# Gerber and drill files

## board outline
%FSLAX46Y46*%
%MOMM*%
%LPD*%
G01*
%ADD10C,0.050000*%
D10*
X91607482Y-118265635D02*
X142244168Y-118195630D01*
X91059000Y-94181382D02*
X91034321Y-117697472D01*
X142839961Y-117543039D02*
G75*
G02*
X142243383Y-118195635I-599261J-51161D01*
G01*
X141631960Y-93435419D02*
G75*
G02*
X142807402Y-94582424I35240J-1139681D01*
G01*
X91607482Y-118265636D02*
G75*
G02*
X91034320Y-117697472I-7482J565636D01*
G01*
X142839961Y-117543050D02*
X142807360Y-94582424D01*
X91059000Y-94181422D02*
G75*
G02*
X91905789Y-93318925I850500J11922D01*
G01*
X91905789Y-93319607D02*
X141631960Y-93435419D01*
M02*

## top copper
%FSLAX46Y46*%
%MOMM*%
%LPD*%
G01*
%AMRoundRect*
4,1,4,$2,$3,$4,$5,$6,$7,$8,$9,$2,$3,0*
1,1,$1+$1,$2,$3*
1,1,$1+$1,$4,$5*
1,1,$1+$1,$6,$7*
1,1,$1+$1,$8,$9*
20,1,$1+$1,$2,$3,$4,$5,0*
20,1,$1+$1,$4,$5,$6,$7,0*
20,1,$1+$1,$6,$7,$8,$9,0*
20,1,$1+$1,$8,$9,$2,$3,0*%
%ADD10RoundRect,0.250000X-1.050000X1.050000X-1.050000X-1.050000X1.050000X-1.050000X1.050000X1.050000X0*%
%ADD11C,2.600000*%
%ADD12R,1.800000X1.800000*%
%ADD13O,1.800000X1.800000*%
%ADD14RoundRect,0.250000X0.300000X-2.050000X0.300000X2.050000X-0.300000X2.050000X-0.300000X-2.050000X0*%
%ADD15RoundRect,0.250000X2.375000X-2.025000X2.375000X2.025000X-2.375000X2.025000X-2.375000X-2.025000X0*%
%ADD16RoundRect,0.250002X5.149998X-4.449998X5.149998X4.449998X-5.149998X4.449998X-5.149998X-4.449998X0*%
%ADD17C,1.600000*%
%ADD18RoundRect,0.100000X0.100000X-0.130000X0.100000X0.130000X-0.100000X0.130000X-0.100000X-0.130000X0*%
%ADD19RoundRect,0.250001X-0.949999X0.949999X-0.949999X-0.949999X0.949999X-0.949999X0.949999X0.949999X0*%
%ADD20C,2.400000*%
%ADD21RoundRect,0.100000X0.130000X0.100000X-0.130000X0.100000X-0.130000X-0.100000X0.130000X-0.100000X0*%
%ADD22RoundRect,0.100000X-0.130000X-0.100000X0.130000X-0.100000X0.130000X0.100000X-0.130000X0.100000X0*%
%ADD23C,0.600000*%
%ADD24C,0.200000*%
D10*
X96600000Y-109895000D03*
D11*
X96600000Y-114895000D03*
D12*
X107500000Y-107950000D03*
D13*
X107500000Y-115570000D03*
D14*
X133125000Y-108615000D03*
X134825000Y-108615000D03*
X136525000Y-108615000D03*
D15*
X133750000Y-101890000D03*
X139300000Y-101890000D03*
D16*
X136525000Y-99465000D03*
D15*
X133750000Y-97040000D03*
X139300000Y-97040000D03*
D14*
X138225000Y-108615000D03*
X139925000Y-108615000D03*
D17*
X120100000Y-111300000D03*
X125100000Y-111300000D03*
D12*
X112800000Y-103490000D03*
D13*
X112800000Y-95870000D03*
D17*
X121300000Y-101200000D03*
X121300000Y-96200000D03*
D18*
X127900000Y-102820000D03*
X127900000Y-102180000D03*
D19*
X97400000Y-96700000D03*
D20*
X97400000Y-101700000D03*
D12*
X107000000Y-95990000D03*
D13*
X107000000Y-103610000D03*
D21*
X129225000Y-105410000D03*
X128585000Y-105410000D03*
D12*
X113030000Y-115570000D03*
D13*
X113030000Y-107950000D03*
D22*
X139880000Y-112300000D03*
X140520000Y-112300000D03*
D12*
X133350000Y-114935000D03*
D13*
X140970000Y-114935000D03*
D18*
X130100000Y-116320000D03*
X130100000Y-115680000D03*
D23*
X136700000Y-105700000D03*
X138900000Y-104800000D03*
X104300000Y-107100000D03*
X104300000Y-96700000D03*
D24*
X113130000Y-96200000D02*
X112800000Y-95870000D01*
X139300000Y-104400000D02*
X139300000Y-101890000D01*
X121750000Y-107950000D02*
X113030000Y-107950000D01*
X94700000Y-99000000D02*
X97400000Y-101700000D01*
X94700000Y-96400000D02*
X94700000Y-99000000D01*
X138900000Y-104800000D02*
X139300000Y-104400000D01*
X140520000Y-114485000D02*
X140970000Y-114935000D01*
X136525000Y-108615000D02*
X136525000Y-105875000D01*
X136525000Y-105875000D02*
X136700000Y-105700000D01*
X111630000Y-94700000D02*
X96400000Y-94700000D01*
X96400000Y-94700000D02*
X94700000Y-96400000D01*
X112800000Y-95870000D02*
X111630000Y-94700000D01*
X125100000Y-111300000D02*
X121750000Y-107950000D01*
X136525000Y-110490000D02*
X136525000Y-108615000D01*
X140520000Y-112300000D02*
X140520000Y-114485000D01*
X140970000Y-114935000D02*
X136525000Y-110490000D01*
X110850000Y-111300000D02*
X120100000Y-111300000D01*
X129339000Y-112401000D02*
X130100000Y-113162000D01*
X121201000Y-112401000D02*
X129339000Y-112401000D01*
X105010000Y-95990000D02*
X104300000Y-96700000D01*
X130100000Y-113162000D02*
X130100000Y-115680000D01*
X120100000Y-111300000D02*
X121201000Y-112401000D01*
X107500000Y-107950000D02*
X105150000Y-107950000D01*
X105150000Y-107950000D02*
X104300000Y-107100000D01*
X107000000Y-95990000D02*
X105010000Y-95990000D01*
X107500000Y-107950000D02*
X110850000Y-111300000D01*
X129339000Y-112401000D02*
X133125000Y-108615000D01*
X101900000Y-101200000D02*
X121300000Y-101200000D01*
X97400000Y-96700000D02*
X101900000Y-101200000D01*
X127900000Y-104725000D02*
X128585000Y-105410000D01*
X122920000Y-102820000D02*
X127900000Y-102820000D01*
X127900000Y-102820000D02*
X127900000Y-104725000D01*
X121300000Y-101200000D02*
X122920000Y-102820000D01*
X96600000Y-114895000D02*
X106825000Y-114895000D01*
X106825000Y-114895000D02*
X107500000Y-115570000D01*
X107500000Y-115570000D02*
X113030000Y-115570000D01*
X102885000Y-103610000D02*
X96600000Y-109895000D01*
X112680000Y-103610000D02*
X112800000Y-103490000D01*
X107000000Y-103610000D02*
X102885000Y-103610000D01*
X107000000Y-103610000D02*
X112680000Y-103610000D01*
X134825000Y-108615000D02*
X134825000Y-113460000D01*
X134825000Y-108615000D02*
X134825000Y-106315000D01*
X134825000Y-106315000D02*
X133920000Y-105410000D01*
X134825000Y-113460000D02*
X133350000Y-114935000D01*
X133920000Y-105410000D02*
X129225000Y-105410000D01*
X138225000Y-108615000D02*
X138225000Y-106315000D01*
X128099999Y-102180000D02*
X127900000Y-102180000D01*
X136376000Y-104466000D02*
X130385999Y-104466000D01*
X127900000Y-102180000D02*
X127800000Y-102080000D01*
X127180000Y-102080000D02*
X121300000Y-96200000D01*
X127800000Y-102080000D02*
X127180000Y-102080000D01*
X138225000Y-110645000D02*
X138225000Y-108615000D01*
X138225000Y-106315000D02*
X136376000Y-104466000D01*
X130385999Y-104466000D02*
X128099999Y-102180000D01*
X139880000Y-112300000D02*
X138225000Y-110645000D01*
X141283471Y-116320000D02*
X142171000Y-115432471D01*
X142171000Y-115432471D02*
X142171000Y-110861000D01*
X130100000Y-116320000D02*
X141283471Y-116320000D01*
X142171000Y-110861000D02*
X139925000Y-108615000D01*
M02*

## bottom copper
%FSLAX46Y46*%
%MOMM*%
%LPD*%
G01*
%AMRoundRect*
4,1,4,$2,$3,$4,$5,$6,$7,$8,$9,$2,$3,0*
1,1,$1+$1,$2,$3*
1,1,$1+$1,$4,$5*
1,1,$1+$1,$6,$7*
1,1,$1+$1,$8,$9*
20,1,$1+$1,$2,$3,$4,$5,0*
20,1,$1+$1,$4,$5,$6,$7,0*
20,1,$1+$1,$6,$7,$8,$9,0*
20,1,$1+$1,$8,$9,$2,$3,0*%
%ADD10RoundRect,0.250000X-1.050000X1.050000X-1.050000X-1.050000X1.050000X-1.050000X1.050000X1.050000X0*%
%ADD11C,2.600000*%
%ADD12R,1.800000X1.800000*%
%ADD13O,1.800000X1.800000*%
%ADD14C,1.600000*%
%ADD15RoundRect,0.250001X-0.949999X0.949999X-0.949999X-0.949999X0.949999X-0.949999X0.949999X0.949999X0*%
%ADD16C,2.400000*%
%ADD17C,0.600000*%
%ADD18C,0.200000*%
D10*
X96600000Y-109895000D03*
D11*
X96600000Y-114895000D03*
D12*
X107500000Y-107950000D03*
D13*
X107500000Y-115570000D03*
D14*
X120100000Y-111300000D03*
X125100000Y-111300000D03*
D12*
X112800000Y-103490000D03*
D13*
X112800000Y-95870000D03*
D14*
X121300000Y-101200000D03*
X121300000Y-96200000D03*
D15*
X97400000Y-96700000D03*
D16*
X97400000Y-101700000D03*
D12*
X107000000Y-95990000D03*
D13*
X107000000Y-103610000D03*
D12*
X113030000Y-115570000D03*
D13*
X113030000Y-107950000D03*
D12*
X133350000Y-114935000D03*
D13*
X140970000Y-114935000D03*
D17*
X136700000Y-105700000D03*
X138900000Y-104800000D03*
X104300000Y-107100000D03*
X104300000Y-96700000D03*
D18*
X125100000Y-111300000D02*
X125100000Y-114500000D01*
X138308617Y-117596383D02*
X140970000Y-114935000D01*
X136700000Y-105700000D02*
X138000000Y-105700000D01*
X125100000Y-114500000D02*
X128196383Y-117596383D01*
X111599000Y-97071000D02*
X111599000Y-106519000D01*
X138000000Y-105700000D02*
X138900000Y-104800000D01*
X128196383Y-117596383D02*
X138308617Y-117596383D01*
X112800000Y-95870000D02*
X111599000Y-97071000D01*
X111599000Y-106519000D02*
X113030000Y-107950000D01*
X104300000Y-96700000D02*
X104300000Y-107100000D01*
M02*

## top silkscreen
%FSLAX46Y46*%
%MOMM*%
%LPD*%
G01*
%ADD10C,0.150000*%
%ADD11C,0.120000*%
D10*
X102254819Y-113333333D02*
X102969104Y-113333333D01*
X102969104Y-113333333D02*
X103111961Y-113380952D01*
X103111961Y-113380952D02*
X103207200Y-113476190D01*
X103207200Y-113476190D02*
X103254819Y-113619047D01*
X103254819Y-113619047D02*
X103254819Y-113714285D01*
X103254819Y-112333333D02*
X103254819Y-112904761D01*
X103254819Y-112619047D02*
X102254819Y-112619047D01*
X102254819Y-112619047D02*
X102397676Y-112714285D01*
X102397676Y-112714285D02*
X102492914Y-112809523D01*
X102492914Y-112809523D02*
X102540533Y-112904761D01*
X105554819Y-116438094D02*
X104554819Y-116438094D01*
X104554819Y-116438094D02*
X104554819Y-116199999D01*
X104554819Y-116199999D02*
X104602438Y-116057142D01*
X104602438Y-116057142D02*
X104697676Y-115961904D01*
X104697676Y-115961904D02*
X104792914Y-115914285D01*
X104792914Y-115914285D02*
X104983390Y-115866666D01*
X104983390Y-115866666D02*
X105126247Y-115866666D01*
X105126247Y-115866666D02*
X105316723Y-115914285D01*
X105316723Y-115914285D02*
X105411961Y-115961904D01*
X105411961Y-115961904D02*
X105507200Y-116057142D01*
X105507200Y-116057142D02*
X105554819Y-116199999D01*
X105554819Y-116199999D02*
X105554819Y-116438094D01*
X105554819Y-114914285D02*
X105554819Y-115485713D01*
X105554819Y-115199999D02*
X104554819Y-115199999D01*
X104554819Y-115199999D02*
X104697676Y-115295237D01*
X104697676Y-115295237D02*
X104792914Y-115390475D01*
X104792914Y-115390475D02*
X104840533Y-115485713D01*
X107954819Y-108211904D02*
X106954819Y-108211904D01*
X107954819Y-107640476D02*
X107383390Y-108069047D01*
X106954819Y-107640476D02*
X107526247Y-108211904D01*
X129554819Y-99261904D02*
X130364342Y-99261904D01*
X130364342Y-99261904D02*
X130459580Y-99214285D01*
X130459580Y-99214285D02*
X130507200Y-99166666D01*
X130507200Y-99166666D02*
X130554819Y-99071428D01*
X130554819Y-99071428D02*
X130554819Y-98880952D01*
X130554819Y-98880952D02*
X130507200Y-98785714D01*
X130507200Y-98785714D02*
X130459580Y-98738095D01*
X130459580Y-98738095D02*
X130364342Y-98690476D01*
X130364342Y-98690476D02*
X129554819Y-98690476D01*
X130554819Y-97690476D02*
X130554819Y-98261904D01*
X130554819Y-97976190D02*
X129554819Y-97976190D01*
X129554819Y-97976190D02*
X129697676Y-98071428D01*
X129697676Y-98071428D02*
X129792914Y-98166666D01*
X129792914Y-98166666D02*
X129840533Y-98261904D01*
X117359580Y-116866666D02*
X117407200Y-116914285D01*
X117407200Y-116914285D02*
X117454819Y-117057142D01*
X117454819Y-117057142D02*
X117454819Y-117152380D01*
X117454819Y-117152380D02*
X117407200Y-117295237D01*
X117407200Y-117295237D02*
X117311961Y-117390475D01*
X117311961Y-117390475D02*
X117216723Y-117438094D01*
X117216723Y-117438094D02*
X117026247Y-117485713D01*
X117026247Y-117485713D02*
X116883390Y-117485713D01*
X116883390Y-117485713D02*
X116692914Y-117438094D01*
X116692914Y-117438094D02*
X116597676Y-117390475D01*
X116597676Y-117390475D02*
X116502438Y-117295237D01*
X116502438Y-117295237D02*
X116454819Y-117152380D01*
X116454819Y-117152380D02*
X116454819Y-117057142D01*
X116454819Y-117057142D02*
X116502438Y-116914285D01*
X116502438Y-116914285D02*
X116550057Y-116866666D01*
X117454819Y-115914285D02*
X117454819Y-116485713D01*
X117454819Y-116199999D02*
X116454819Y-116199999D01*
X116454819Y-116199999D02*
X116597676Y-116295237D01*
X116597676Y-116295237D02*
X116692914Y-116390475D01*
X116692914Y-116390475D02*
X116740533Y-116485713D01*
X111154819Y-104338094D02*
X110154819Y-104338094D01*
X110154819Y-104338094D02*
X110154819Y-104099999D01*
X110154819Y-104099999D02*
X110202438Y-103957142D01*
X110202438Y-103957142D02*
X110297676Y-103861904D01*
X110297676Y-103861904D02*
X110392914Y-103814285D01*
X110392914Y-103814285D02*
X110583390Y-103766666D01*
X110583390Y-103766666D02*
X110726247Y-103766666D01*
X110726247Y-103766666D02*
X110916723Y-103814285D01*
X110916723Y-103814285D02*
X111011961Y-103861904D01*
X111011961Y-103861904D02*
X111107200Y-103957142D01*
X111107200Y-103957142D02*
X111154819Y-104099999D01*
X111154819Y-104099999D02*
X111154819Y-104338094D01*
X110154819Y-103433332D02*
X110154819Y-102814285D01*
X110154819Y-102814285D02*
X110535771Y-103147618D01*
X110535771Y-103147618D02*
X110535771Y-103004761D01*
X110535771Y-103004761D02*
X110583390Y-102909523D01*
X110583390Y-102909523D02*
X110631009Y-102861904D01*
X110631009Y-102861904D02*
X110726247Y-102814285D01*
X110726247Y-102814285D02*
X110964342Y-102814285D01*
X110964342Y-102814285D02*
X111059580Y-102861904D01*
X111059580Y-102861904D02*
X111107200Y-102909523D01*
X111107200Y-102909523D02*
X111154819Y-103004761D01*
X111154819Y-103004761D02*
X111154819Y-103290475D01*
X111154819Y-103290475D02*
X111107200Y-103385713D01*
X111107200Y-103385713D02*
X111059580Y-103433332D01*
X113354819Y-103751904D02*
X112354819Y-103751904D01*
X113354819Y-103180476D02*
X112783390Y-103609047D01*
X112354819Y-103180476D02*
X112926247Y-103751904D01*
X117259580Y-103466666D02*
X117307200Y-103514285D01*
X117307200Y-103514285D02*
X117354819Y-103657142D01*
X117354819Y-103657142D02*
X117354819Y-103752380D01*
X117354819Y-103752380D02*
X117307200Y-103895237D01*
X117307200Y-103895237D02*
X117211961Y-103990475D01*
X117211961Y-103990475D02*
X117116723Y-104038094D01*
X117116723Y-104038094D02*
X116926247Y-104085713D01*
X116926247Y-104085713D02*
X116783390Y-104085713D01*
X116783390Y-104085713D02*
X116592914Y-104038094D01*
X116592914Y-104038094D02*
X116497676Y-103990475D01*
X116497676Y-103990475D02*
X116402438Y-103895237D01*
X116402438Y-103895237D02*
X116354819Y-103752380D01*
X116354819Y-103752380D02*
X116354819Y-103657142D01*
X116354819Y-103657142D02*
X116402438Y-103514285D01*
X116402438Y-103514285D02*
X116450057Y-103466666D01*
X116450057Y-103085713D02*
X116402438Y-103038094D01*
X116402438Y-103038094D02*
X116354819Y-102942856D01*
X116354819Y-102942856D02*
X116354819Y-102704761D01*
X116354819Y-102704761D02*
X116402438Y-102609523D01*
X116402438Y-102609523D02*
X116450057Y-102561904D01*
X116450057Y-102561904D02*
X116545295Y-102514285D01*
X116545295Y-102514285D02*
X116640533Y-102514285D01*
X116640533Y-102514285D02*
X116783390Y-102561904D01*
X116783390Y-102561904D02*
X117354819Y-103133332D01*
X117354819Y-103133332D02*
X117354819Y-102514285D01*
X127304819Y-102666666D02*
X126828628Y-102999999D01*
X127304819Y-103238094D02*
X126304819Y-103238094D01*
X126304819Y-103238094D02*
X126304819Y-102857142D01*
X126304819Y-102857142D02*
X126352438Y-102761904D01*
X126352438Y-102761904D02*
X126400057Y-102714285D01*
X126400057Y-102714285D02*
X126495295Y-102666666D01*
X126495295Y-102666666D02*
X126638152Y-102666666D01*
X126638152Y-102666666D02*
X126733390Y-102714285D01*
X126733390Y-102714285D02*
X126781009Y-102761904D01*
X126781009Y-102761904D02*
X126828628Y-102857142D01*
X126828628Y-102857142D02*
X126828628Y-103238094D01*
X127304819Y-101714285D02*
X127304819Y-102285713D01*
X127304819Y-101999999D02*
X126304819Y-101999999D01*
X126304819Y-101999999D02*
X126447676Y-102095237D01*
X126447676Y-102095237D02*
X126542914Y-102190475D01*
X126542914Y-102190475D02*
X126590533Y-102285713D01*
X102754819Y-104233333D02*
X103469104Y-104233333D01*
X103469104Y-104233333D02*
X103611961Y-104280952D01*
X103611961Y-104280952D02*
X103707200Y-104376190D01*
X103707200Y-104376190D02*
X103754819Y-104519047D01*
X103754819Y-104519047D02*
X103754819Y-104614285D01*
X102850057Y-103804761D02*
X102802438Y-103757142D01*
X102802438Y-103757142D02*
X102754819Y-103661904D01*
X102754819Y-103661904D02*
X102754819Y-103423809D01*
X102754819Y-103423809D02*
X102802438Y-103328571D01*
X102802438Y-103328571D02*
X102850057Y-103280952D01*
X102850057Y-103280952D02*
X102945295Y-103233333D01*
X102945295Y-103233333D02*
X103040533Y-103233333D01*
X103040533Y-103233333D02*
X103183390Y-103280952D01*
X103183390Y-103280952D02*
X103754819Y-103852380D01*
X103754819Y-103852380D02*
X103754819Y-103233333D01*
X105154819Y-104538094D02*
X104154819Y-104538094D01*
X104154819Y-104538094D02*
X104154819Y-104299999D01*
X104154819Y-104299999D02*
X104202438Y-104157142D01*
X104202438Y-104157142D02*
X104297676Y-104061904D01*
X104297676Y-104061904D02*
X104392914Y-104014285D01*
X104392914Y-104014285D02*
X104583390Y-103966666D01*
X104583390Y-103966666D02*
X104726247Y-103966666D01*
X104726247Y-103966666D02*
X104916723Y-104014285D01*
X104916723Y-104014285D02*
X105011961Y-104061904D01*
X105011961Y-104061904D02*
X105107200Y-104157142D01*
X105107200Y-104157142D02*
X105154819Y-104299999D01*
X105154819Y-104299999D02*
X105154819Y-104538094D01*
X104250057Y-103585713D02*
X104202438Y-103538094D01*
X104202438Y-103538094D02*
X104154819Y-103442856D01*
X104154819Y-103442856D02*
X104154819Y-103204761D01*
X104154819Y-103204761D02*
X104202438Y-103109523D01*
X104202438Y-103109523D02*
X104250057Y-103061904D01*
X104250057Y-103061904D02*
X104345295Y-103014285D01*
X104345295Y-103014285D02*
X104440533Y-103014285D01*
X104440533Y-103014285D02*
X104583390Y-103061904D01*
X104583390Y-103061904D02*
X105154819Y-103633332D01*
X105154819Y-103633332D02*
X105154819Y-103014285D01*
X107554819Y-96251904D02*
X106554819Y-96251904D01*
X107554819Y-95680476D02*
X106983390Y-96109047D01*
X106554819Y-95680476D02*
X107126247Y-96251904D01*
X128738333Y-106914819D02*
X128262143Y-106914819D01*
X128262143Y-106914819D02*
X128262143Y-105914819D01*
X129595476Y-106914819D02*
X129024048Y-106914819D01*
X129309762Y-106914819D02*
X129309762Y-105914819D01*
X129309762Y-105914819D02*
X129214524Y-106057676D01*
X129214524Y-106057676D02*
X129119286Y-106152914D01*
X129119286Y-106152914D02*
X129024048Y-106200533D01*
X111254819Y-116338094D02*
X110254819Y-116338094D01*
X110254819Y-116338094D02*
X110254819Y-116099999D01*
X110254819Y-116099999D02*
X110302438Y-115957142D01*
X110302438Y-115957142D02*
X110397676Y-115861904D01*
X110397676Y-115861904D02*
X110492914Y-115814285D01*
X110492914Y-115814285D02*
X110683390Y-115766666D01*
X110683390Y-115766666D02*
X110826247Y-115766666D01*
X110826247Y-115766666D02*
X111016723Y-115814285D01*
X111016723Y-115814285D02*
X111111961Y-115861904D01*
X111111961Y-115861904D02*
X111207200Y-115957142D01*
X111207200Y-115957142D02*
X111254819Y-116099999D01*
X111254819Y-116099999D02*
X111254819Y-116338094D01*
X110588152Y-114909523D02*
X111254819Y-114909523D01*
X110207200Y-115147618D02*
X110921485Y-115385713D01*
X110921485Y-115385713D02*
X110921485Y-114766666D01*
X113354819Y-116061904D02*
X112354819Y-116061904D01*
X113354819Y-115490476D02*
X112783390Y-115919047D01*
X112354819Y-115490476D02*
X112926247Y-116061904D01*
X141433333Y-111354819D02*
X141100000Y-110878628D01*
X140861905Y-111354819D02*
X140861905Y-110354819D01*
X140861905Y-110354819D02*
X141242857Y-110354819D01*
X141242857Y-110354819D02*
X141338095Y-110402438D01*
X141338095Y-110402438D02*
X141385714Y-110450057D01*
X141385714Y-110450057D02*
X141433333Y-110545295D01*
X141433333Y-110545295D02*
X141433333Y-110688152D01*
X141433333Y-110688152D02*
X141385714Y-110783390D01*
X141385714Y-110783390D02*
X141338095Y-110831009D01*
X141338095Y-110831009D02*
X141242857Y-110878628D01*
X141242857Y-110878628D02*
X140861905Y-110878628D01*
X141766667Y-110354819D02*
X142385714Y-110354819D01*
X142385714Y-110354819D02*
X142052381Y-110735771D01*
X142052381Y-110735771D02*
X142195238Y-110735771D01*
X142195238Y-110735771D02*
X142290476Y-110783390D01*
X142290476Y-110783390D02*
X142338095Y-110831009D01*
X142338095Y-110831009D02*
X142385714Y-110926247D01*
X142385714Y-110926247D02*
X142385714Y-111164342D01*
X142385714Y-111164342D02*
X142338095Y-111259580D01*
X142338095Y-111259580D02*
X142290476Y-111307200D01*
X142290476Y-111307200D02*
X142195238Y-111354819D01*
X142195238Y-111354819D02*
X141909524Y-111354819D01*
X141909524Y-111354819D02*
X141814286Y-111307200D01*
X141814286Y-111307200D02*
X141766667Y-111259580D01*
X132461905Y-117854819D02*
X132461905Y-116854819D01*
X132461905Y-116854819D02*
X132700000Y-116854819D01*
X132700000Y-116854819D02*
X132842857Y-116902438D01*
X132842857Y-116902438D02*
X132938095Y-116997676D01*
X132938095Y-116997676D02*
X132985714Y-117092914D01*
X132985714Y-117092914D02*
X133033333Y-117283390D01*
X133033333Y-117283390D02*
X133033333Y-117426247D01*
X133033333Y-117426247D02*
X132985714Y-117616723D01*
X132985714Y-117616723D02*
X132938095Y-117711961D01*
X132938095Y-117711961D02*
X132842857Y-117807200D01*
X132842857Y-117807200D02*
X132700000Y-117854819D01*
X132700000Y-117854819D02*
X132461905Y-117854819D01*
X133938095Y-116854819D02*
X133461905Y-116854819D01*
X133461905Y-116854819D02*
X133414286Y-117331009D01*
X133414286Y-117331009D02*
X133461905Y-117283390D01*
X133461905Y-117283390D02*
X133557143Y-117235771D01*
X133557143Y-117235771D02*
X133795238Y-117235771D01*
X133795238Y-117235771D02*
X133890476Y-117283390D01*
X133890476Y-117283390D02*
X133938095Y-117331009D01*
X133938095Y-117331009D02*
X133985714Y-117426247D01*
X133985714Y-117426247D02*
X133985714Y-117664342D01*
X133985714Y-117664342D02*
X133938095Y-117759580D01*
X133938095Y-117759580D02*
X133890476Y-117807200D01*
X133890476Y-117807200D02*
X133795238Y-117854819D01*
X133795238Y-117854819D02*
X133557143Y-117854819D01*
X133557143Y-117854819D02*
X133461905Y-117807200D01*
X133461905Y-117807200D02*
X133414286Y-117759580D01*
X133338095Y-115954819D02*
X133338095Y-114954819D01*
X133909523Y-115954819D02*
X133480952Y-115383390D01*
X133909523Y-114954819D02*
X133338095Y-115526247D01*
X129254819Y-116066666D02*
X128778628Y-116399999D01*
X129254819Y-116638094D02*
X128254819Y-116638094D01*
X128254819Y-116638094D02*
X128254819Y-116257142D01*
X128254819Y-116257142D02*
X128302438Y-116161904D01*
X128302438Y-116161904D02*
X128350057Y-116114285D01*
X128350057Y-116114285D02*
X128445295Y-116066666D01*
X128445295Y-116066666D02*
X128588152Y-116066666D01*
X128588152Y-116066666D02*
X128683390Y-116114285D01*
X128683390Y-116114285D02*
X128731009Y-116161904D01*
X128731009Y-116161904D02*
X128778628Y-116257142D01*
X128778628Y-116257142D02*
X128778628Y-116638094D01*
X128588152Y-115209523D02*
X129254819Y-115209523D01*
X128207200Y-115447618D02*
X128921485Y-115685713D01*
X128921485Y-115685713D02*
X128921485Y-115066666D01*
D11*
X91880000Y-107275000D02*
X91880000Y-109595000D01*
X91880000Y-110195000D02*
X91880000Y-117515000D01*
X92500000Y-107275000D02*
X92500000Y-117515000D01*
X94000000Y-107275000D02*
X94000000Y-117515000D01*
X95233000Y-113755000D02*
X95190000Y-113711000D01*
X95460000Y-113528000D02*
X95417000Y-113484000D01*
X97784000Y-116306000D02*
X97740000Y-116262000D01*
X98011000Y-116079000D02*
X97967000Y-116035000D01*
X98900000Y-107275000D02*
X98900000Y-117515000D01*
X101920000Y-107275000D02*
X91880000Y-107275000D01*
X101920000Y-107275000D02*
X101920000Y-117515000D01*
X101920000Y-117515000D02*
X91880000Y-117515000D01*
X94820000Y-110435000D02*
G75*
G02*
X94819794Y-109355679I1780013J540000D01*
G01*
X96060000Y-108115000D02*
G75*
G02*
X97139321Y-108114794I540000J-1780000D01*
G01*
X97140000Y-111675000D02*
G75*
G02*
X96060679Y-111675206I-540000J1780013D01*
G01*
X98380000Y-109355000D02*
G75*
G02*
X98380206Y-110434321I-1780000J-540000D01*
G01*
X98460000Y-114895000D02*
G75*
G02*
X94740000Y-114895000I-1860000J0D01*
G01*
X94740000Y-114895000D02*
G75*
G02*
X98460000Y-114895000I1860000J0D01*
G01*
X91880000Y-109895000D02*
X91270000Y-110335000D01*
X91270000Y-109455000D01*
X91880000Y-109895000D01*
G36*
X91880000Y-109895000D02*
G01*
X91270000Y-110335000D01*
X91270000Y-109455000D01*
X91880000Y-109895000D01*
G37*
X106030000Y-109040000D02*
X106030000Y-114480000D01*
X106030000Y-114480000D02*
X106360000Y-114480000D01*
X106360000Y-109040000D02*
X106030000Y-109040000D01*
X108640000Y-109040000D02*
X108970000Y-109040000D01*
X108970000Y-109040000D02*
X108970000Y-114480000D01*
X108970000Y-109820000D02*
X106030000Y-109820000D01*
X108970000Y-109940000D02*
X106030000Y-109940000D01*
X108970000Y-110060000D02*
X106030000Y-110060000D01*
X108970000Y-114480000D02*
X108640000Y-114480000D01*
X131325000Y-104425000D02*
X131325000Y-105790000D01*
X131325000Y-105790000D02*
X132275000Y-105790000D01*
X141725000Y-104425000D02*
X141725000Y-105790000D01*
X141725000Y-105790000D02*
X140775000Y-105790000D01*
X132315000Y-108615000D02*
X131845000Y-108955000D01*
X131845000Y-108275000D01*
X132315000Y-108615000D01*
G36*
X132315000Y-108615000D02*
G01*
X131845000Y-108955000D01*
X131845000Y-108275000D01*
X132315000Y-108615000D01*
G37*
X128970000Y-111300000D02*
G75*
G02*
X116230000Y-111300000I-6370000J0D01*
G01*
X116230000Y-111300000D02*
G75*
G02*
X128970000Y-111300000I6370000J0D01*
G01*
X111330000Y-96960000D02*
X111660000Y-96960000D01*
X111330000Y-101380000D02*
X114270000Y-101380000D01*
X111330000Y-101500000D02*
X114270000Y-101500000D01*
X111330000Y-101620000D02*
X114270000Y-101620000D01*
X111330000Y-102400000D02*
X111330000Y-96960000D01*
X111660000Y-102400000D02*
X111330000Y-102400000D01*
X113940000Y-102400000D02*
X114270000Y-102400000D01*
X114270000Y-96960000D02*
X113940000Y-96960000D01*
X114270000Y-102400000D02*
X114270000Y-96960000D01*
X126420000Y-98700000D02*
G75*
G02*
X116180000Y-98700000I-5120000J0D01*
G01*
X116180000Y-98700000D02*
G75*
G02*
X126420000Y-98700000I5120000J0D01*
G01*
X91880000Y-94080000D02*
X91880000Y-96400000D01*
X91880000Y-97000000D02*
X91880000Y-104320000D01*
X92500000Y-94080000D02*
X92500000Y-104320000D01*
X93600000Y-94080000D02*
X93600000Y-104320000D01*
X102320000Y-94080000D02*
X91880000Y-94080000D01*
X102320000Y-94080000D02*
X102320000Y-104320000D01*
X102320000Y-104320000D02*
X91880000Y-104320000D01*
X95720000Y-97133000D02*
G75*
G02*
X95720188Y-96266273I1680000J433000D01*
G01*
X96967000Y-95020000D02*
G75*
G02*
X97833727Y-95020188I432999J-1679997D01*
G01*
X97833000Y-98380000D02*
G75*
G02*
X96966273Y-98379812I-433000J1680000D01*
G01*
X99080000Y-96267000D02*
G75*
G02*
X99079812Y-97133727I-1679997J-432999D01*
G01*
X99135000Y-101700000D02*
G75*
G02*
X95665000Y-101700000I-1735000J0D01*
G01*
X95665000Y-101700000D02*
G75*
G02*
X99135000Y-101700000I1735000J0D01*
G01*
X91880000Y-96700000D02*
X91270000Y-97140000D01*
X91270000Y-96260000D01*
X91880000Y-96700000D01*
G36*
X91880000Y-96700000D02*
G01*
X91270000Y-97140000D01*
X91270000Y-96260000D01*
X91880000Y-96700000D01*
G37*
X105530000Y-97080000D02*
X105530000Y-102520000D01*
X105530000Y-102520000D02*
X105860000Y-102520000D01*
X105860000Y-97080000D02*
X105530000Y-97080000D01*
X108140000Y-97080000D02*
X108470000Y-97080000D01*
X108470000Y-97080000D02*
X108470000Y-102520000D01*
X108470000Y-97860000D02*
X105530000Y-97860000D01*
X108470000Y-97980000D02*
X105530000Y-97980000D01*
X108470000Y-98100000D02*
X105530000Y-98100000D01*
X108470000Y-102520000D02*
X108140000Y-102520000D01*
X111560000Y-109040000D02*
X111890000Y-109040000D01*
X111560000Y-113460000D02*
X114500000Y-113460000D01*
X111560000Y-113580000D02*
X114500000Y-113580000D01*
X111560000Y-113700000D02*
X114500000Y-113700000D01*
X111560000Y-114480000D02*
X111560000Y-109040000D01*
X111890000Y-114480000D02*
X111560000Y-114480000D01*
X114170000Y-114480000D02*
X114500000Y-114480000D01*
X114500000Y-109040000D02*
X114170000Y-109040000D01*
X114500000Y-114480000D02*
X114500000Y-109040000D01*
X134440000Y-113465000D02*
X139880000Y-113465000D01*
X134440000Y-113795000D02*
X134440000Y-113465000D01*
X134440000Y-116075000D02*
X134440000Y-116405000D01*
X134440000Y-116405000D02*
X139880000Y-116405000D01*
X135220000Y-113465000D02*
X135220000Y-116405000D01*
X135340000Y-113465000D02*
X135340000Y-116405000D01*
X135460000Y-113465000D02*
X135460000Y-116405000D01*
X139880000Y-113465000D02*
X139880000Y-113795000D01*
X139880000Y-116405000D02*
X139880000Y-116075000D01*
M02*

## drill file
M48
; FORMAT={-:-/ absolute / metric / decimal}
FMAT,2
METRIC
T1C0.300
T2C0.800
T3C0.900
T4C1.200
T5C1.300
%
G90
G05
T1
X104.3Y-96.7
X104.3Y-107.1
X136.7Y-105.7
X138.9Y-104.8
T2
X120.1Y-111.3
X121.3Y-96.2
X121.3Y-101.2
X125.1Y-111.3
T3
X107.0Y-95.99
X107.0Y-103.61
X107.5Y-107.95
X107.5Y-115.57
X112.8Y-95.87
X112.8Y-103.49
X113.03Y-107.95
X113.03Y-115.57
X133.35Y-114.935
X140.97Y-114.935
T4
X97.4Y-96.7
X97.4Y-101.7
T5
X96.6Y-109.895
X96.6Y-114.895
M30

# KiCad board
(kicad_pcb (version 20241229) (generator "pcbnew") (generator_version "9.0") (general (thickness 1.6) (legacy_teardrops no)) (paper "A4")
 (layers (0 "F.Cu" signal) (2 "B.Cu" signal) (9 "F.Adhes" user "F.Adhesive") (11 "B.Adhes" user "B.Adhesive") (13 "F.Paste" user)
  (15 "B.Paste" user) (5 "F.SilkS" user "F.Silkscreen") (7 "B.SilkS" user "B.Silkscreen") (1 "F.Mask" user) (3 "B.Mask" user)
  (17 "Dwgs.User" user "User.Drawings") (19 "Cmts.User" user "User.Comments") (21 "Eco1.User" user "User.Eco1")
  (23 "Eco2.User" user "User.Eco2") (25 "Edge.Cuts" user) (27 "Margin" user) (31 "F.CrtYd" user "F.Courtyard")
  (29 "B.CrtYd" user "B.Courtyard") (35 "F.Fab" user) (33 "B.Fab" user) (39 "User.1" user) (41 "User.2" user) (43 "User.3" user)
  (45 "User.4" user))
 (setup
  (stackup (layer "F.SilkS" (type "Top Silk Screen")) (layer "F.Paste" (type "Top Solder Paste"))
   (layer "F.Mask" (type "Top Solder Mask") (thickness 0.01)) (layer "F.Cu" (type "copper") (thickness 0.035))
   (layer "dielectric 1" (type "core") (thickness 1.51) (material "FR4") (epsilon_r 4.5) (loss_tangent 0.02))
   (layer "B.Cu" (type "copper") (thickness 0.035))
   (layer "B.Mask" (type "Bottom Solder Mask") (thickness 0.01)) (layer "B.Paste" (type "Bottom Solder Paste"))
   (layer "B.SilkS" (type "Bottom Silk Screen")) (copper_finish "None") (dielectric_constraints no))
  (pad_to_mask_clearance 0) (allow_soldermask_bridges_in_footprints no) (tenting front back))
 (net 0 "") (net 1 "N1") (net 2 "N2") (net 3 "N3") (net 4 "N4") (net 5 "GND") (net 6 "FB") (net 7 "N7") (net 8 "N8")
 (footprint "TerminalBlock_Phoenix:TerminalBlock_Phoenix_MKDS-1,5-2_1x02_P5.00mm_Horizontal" (layer "F.Cu") (at 96.6 109.895 -90)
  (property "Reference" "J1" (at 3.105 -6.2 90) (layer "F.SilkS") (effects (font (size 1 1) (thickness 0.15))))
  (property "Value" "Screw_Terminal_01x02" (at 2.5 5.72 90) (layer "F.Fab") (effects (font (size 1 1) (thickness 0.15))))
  (fp_line (start -2.62 4.72) (end -0.3 4.72) (stroke (width 0.12) (type solid)) (layer "F.SilkS"))
  (fp_line (start 0.3 4.72) (end 7.62 4.72) (stroke (width 0.12) (type solid)) (layer "F.SilkS"))
  (fp_line (start -2.62 4.1) (end 7.62 4.1) (stroke (width 0.12) (type solid)) (layer "F.SilkS"))
  (fp_line (start -2.62 2.6) (end 7.62 2.6) (stroke (width 0.12) (type solid)) (layer "F.SilkS"))
  (fp_line (start 3.86 1.367) (end 3.816 1.41) (stroke (width 0.12) (type solid)) (layer "F.SilkS"))
  (fp_line (start 3.633 1.14) (end 3.589 1.183) (stroke (width 0.12) (type solid)) (layer "F.SilkS"))
  (fp_line (start 6.411 -1.184) (end 6.367 -1.14) (stroke (width 0.12) (type solid)) (layer "F.SilkS"))
  (fp_line (start 6.184 -1.411) (end 6.14 -1.367) (stroke (width 0.12) (type solid)) (layer "F.SilkS"))
  (fp_line (start -2.62 -2.3) (end 7.62 -2.3) (stroke (width 0.12) (type solid)) (layer "F.SilkS"))
  (fp_line (start -2.62 -5.32) (end -2.62 4.72) (stroke (width 0.12) (type solid)) (layer "F.SilkS"))
  (fp_line (start -2.62 -5.32) (end 7.62 -5.32) (stroke (width 0.12) (type solid)) (layer "F.SilkS"))
  (fp_line (start 7.62 -5.32) (end 7.62 4.72) (stroke (width 0.12) (type solid)) (layer "F.SilkS"))
  (fp_arc (start 0.54 1.78) (mid 0.000355 1.860107) (end -0.539321 1.780206) (stroke (width 0.12) (type solid)) (layer "F.SilkS"))
  (fp_arc (start -1.78 0.54) (mid -1.860107 0.000355) (end -1.780206 -0.539321) (stroke (width 0.12) (type solid)) (layer "F.SilkS"))
  (fp_arc (start 1.78 -0.54) (mid 1.860107 -0.000355) (end 1.780206 0.539321) (stroke (width 0.12) (type solid)) (layer "F.SilkS"))
  (fp_arc (start -0.54 -1.78) (mid -0.000355 -1.860107) (end 0.539321 -1.780206) (stroke (width 0.12) (type solid)) (layer "F.SilkS"))
  (fp_circle (center 5 0) (end 6.86 0) (stroke (width 0.12) (type solid)) (fill no) (layer "F.SilkS"))
  (fp_poly (pts (xy 0 4.72) (xy 0.44 5.33) (xy -0.44 5.33) (xy 0 4.72)) (stroke (width 0.12) (type solid)) (fill yes) (layer "F.SilkS"))
  (pad "1" thru_hole roundrect (at 0 0 270) (size 2.6 2.6) (drill 1.3) (layers "*.Cu" "*.Mask") (remove_unused_layers no)
   (roundrect_rratio 0.096154) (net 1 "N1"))
  (pad "2" thru_hole circle (at 5 0 270) (size 2.6 2.6) (drill 1.3) (layers "*.Cu" "*.Mask") (remove_unused_layers no) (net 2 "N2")))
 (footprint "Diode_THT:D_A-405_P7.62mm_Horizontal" (layer "F.Cu") (at 107.5 107.95 -90)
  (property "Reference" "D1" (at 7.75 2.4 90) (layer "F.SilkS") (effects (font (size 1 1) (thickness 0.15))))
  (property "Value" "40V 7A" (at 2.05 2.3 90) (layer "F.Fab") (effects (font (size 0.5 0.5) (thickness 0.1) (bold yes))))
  (fp_line (start 1.09 1.47) (end 6.53 1.47) (stroke (width 0.12) (type solid)) (layer "F.SilkS"))
  (fp_line (start 6.53 1.47) (end 6.53 1.14) (stroke (width 0.12) (type solid)) (layer "F.SilkS"))
  (fp_line (start 1.09 1.14) (end 1.09 1.47) (stroke (width 0.12) (type solid)) (layer "F.SilkS"))
  (fp_line (start 1.09 -1.14) (end 1.09 -1.47) (stroke (width 0.12) (type solid)) (layer "F.SilkS"))
  (fp_line (start 1.09 -1.47) (end 6.53 -1.47) (stroke (width 0.12) (type solid)) (layer "F.SilkS"))
  (fp_line (start 1.87 -1.47) (end 1.87 1.47) (stroke (width 0.12) (type solid)) (layer "F.SilkS"))
  (fp_line (start 1.99 -1.47) (end 1.99 1.47) (stroke (width 0.12) (type solid)) (layer "F.SilkS"))
  (fp_line (start 2.11 -1.47) (end 2.11 1.47) (stroke (width 0.12) (type solid)) (layer "F.SilkS"))
  (fp_line (start 6.53 -1.47) (end 6.53 -1.14) (stroke (width 0.12) (type solid)) (layer "F.SilkS"))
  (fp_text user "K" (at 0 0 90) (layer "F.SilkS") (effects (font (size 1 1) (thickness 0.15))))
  (pad "1" thru_hole rect (at 0 0 270) (size 1.8 1.8) (drill 0.9) (layers "*.Cu" "*.Mask") (remove_unused_layers no) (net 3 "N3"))
  (pad "2" thru_hole oval (at 7.62 0 270) (size 1.8 1.8) (drill 0.9) (layers "*.Cu" "*.Mask") (remove_unused_layers no) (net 2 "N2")))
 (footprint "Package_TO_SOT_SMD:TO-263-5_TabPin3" (layer "F.Cu") (at 136.525 100.965 90)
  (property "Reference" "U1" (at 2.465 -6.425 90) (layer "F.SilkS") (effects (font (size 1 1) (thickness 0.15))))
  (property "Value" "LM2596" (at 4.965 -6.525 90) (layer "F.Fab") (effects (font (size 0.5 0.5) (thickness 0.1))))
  (fp_line (start -3.46 -5.2) (end -4.825 -5.2) (stroke (width 0.12) (type solid)) (layer "F.SilkS"))
  (fp_line (start -4.825 -5.2) (end -4.825 -4.25) (stroke (width 0.12) (type solid)) (layer "F.SilkS"))
  (fp_line (start -3.46 5.2) (end -4.825 5.2) (stroke (width 0.12) (type solid)) (layer "F.SilkS"))
  (fp_line (start -4.825 5.2) (end -4.825 4.25) (stroke (width 0.12) (type solid)) (layer "F.SilkS"))
  (fp_poly
   (pts (xy -7.65 -4.21) (xy -7.99 -4.68) (xy -7.31 -4.68) (xy -7.65 -4.21)) (stroke (width 0.12) (type solid)) (fill yes) (layer "F.SilkS"))
  (pad "1" smd roundrect (at -7.65 -3.4 90) (size 4.6 1.1) (layers "F.Cu" "F.Mask" "F.Paste") (roundrect_rratio 0.227273) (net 3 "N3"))
  (pad "2" smd roundrect (at -7.65 -1.7 90) (size 4.6 1.1) (layers "F.Cu" "F.Mask" "F.Paste") (roundrect_rratio 0.227273) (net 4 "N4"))
  (pad "3" smd roundrect (at -7.65 0 90) (size 4.6 1.1) (layers "F.Cu" "F.Mask" "F.Paste") (roundrect_rratio 0.227273) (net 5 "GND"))
  (pad "3" smd roundrect (at -0.925 -2.775 90) (size 4.55 5.25) (layers "F.Cu" "F.Paste") (roundrect_rratio 0.054945) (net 5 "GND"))
  (pad "3" smd roundrect (at -0.925 2.775 90) (size 4.55 5.25) (layers "F.Cu" "F.Paste") (roundrect_rratio 0.054945) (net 5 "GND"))
  (pad "3" smd roundrect (at 1.5 0 90) (size 9.4 10.8) (layers "F.Cu" "F.Mask") (roundrect_rratio 0.026596) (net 5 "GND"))
  (pad "3" smd roundrect (at 3.925 -2.775 90) (size 4.55 5.25) (layers "F.Cu" "F.Paste") (roundrect_rratio 0.054945) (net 5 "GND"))
  (pad "3" smd roundrect (at 3.925 2.775 90) (size 4.55 5.25) (layers "F.Cu" "F.Paste") (roundrect_rratio 0.054945) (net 5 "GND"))
  (pad "4" smd roundrect (at -7.65 1.7 90) (size 4.6 1.1) (layers "F.Cu" "F.Mask" "F.Paste") (roundrect_rratio 0.227273) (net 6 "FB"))
  (pad "5" smd roundrect (at -7.65 3.4 90) (size 4.6 1.1) (layers "F.Cu" "F.Mask" "F.Paste") (roundrect_rratio 0.227273) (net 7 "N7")))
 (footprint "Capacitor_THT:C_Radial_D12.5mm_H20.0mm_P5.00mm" (layer "F.Cu") (at 120.1 111.3)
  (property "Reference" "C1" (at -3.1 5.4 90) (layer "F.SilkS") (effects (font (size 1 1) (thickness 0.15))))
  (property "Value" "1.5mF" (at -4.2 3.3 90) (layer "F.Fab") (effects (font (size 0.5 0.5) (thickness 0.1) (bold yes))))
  (fp_circle (center 2.5 0) (end 8.87 0) (stroke (width 0.12) (type solid)) (fill no) (layer "F.SilkS"))
  (pad "1" thru_hole circle (at 0 0) (size 1.6 1.6) (drill 0.8) (layers "*.Cu" "*.Mask") (remove_unused_layers no) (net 3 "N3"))
  (pad "2" thru_hole circle (at 5 0) (size 1.6 1.6) (drill 0.8) (layers "*.Cu" "*.Mask") (remove_unused_layers no) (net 5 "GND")))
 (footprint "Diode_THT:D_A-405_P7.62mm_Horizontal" (layer "F.Cu") (at 112.8 103.49 90)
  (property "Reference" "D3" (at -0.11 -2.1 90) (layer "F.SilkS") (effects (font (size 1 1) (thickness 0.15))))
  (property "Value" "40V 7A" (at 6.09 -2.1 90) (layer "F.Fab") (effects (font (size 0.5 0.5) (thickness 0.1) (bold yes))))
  (fp_line (start 6.53 -1.47) (end 6.53 -1.14) (stroke (width 0.12) (type solid)) (layer "F.SilkS"))
  (fp_line (start 2.11 -1.47) (end 2.11 1.47) (stroke (width 0.12) (type solid)) (layer "F.SilkS"))
  (fp_line (start 1.99 -1.47) (end 1.99 1.47) (stroke (width 0.12) (type solid)) (layer "F.SilkS"))
  (fp_line (start 1.87 -1.47) (end 1.87 1.47) (stroke (width 0.12) (type solid)) (layer "F.SilkS"))
  (fp_line (start 1.09 -1.47) (end 6.53 -1.47) (stroke (width 0.12) (type solid)) (layer "F.SilkS"))
  (fp_line (start 1.09 -1.14) (end 1.09 -1.47) (stroke (width 0.12) (type solid)) (layer "F.SilkS"))
  (fp_line (start 1.09 1.14) (end 1.09 1.47) (stroke (width 0.12) (type solid)) (layer "F.SilkS"))
  (fp_line (start 6.53 1.47) (end 6.53 1.14) (stroke (width 0.12) (type solid)) (layer "F.SilkS"))
  (fp_line (start 1.09 1.47) (end 6.53 1.47) (stroke (width 0.12) (type solid)) (layer "F.SilkS"))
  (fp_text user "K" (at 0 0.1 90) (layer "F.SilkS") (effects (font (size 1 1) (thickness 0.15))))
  (pad "1" thru_hole rect (at 0 0 90) (size 1.8 1.8) (drill 0.9) (layers "*.Cu" "*.Mask") (remove_unused_layers no) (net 1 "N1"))
  (pad "2" thru_hole oval (at 7.62 0 90) (size 1.8 1.8) (drill 0.9) (layers "*.Cu" "*.Mask") (remove_unused_layers no) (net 5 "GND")))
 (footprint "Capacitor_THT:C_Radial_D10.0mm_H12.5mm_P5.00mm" (layer "F.Cu") (at 121.3 101.2 90)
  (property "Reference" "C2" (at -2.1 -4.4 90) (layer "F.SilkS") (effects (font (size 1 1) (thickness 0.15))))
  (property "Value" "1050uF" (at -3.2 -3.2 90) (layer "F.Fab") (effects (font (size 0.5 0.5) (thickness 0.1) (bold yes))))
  (fp_circle (center 2.5 0) (end 7.62 0) (stroke (width 0.12) (type solid)) (fill no) (layer "F.SilkS"))
  (pad "1" thru_hole circle (at 0 0 90) (size 1.6 1.6) (drill 0.8) (layers "*.Cu" "*.Mask") (remove_unused_layers no) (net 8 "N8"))
  (pad "2" thru_hole circle (at 5 0 90) (size 1.6 1.6) (drill 0.8) (layers "*.Cu" "*.Mask") (remove_unused_layers no) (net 6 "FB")))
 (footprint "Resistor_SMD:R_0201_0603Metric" (layer "F.Cu") (at 127.9 102.5 90)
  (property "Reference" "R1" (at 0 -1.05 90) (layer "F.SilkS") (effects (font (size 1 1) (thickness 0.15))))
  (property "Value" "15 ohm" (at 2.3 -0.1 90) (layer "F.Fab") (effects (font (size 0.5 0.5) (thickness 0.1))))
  (pad "" smd roundrect (at -0.345 0 90) (size 0.318 0.36) (layers "F.Paste") (roundrect_rratio 0.25))
  (pad "" smd roundrect (at 0.345 0 90) (size 0.318 0.36) (layers "F.Paste") (roundrect_rratio 0.25))
  (pad "1" smd roundrect (at -0.32 0 90) (size 0.46 0.4) (layers "F.Cu" "F.Mask") (roundrect_rratio 0.25) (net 8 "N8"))
  (pad "2" smd roundrect (at 0.32 0 90) (size 0.46 0.4) (layers "F.Cu" "F.Mask") (roundrect_rratio 0.25) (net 6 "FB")))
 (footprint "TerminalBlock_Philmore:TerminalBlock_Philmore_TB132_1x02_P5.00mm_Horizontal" (layer "F.Cu") (at 97.4 96.7 -90)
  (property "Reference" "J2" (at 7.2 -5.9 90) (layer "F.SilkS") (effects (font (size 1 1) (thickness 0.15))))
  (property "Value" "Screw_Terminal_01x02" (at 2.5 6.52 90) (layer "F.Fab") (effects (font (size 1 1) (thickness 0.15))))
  (fp_line (start -2.62 5.52) (end -0.3 5.52) (stroke (width 0.12) (type solid)) (layer "F.SilkS"))
  (fp_line (start 0.3 5.52) (end 7.62 5.52) (stroke (width 0.12) (type solid)) (layer "F.SilkS"))
  (fp_line (start -2.62 4.9) (end 7.62 4.9) (stroke (width 0.12) (type solid)) (layer "F.SilkS"))
  (fp_line (start -2.62 3.8) (end 7.62 3.8) (stroke (width 0.12) (type solid)) (layer "F.SilkS"))
  (fp_line (start -2.62 -4.92) (end -2.62 5.52) (stroke (width 0.12) (type solid)) (layer "F.SilkS"))
  (fp_line (start -2.62 -4.92) (end 7.62 -4.92) (stroke (width 0.12) (type solid)) (layer "F.SilkS"))
  (fp_line (start 7.62 -4.92) (end 7.62 5.52) (stroke (width 0.12) (type solid)) (layer "F.SilkS"))
  (fp_arc (start 0.433 1.68) (mid -0.000376 1.734903) (end -0.433727 1.679812) (stroke (width 0.12) (type solid)) (layer "F.SilkS"))
  (fp_arc (start -1.68 0.433) (mid -1.734903 -0.000376) (end -1.679812 -0.433727) (stroke (width 0.12) (type solid)) (layer "F.SilkS"))
  (fp_arc (start 1.68 -0.433) (mid 1.734903 0.000376) (end 1.679812 0.433727) (stroke (width 0.12) (type solid)) (layer "F.SilkS"))
  (fp_arc (start -0.433 -1.68) (mid 0.000376 -1.734903) (end 0.433727 -1.679812) (stroke (width 0.12) (type solid)) (layer "F.SilkS"))
  (fp_circle (center 5 0) (end 6.735 0) (stroke (width 0.12) (type solid)) (fill no) (layer "F.SilkS"))
  (fp_poly (pts (xy 0 5.52) (xy 0.44 6.13) (xy -0.44 6.13) (xy 0 5.52)) (stroke (width 0.12) (type solid)) (fill yes) (layer "F.SilkS"))
  (pad "1" thru_hole roundrect (at 0 0 270) (size 2.4 2.4) (drill 1.2) (layers "*.Cu" "*.Mask") (remove_unused_layers no)
   (roundrect_rratio 0.104167) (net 8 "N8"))
  (pad "2" thru_hole circle (at 5 0 270) (size 2.4 2.4) (drill 1.2) (layers "*.Cu" "*.Mask") (remove_unused_layers no) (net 5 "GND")))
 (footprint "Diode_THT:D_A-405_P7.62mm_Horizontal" (layer "F.Cu") (at 107 95.99 -90)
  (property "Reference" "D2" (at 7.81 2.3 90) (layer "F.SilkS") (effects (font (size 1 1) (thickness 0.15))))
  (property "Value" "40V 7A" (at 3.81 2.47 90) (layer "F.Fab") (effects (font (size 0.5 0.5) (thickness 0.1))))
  (fp_line (start 1.09 1.47) (end 6.53 1.47) (stroke (width 0.12) (type solid)) (layer "F.SilkS"))
  (fp_line (start 6.53 1.47) (end 6.53 1.14) (stroke (width 0.12) (type solid)) (layer "F.SilkS"))
  (fp_line (start 1.09 1.14) (end 1.09 1.47) (stroke (width 0.12) (type solid)) (layer "F.SilkS"))
  (fp_line (start 1.09 -1.14) (end 1.09 -1.47) (stroke (width 0.12) (type solid)) (layer "F.SilkS"))
  (fp_line (start 1.09 -1.47) (end 6.53 -1.47) (stroke (width 0.12) (type solid)) (layer "F.SilkS"))
  (fp_line (start 1.87 -1.47) (end 1.87 1.47) (stroke (width 0.12) (type solid)) (layer "F.SilkS"))
  (fp_line (start 1.99 -1.47) (end 1.99 1.47) (stroke (width 0.12) (type solid)) (layer "F.SilkS"))
  (fp_line (start 2.11 -1.47) (end 2.11 1.47) (stroke (width 0.12) (type solid)) (layer "F.SilkS"))
  (fp_line (start 6.53 -1.47) (end 6.53 -1.14) (stroke (width 0.12) (type solid)) (layer "F.SilkS"))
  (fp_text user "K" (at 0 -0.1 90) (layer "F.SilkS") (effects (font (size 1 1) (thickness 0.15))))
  (pad "1" thru_hole rect (at 0 0 270) (size 1.8 1.8) (drill 0.9) (layers "*.Cu" "*.Mask") (remove_unused_layers no) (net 3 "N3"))
  (pad "2" thru_hole oval (at 7.62 0 270) (size 1.8 1.8) (drill 0.9) (layers "*.Cu" "*.Mask") (remove_unused_layers no) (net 1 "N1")))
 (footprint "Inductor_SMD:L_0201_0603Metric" (layer "F.Cu") (at 128.905 105.41 180)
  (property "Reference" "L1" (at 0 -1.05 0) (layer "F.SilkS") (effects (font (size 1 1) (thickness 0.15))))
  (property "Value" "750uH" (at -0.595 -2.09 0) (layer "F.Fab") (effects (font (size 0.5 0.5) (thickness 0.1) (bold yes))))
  (pad "" smd roundrect (at -0.345 0 180) (size 0.318 0.36) (layers "F.Paste") (roundrect_rratio 0.25))
  (pad "" smd roundrect (at 0.345 0 180) (size 0.318 0.36) (layers "F.Paste") (roundrect_rratio 0.25))
  (pad "1" smd roundrect (at -0.32 0 180) (size 0.46 0.4) (layers "F.Cu" "F.Mask") (roundrect_rratio 0.25) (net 4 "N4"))
  (pad "2" smd roundrect (at 0.32 0 180) (size 0.46 0.4) (layers "F.Cu" "F.Mask") (roundrect_rratio 0.25) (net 8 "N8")))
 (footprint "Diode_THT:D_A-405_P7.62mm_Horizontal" (layer "F.Cu") (at 113.03 115.57 90)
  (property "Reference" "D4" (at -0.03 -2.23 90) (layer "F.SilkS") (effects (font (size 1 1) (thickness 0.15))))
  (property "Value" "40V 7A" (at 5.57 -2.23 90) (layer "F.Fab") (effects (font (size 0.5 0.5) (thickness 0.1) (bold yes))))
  (fp_line (start 6.53 -1.47) (end 6.53 -1.14) (stroke (width 0.12) (type solid)) (layer "F.SilkS"))
  (fp_line (start 2.11 -1.47) (end 2.11 1.47) (stroke (width 0.12) (type solid)) (layer "F.SilkS"))
  (fp_line (start 1.99 -1.47) (end 1.99 1.47) (stroke (width 0.12) (type solid)) (layer "F.SilkS"))
  (fp_line (start 1.87 -1.47) (end 1.87 1.47) (stroke (width 0.12) (type solid)) (layer "F.SilkS"))
  (fp_line (start 1.09 -1.47) (end 6.53 -1.47) (stroke (width 0.12) (type solid)) (layer "F.SilkS"))
  (fp_line (start 1.09 -1.14) (end 1.09 -1.47) (stroke (width 0.12) (type solid)) (layer "F.SilkS"))
  (fp_line (start 1.09 1.14) (end 1.09 1.47) (stroke (width 0.12) (type solid)) (layer "F.SilkS"))
  (fp_line (start 6.53 1.47) (end 6.53 1.14) (stroke (width 0.12) (type solid)) (layer "F.SilkS"))
  (fp_line (start 1.09 1.47) (end 6.53 1.47) (stroke (width 0.12) (type solid)) (layer "F.SilkS"))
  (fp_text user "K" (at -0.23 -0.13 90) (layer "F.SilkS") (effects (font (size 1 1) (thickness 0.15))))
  (pad "1" thru_hole rect (at 0 0 90) (size 1.8 1.8) (drill 0.9) (layers "*.Cu" "*.Mask") (remove_unused_layers no) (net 2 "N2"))
  (pad "2" thru_hole oval (at 7.62 0 90) (size 1.8 1.8) (drill 0.9) (layers "*.Cu" "*.Mask") (remove_unused_layers no) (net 5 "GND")))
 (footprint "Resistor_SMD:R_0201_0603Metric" (layer "F.Cu") (at 140.2 112.3)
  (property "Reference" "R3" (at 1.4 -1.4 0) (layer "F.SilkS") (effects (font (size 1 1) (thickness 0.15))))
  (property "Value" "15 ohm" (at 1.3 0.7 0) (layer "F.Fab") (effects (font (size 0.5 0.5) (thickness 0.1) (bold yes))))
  (pad "" smd roundrect (at -0.345 0) (size 0.318 0.36) (layers "F.Paste") (roundrect_rratio 0.25))
  (pad "" smd roundrect (at 0.345 0) (size 0.318 0.36) (layers "F.Paste") (roundrect_rratio 0.25))
  (pad "1" smd roundrect (at -0.32 0) (size 0.46 0.4) (layers "F.Cu" "F.Mask") (roundrect_rratio 0.25) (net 6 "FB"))
  (pad "2" smd roundrect (at 0.32 0) (size 0.46 0.4) (layers "F.Cu" "F.Mask") (roundrect_rratio 0.25) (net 5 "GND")))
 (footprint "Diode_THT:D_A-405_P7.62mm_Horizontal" (layer "F.Cu") (at 133.35 114.935)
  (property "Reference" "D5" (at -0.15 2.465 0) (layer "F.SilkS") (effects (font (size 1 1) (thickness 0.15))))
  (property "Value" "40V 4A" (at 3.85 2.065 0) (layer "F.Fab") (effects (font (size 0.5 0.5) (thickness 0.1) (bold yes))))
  (fp_line (start 1.09 -1.47) (end 6.53 -1.47) (stroke (width 0.12) (type solid)) (layer "F.SilkS"))
  (fp_line (start 1.09 -1.14) (end 1.09 -1.47) (stroke (width 0.12) (type solid)) (layer "F.SilkS"))
  (fp_line (start 1.09 1.14) (end 1.09 1.47) (stroke (width 0.12) (type solid)) (layer "F.SilkS"))
  (fp_line (start 1.09 1.47) (end 6.53 1.47) (stroke (width 0.12) (type solid)) (layer "F.SilkS"))
  (fp_line (start 1.87 -1.47) (end 1.87 1.47) (stroke (width 0.12) (type solid)) (layer "F.SilkS"))
  (fp_line (start 1.99 -1.47) (end 1.99 1.47) (stroke (width 0.12) (type solid)) (layer "F.SilkS"))
  (fp_line (start 2.11 -1.47) (end 2.11 1.47) (stroke (width 0.12) (type solid)) (layer "F.SilkS"))
  (fp_line (start 6.53 -1.47) (end 6.53 -1.14) (stroke (width 0.12) (type solid)) (layer "F.SilkS"))
  (fp_line (start 6.53 1.47) (end 6.53 1.14) (stroke (width 0.12) (type solid)) (layer "F.SilkS"))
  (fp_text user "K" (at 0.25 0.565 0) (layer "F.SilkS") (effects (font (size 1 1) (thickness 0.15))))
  (pad "1" thru_hole rect (at 0 0) (size 1.8 1.8) (drill 0.9) (layers "*.Cu" "*.Mask") (remove_unused_layers no) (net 4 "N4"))
  (pad "2" thru_hole oval (at 7.62 0) (size 1.8 1.8) (drill 0.9) (layers "*.Cu" "*.Mask") (remove_unused_layers no) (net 5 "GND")))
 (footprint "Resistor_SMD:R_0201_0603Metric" (layer "F.Cu") (at 130.1 116 90)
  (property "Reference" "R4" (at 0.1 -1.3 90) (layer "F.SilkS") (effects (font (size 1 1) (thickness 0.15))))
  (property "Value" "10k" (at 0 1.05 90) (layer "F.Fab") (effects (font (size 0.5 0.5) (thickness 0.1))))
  (pad "" smd roundrect (at -0.345 0 90) (size 0.318 0.36) (layers "F.Paste") (roundrect_rratio 0.25))
  (pad "" smd roundrect (at 0.345 0 90) (size 0.318 0.36) (layers "F.Paste") (roundrect_rratio 0.25))
  (pad "1" smd roundrect (at -0.32 0 90) (size 0.46 0.4) (layers "F.Cu" "F.Mask") (roundrect_rratio 0.25) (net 7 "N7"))
  (pad "2" smd roundrect (at 0.32 0 90) (size 0.46 0.4) (layers "F.Cu" "F.Mask") (roundrect_rratio 0.25) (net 3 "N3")))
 (gr_line (start 91.607482 118.265635) (end 142.244168 118.19563) (stroke (width 0.05) (type default)) (layer "Edge.Cuts"))
 (gr_line (start 91.059 94.181382) (end 91.034321 117.697472) (stroke (width 0.05) (type default)) (layer "Edge.Cuts"))
 (gr_arc (start 142.839961 117.543039) (mid 142.684606 118) (end 142.243383 118.19563) (stroke (width 0.05) (type default))
  (layer "Edge.Cuts"))
 (gr_arc (start 141.63196 93.435419) (mid 142.463516 93.759029) (end 142.80736 94.582424) (stroke (width 0.05) (type default))
  (layer "Edge.Cuts"))
 (gr_arc (start 91.607482 118.265636) (mid 91.201755 118.101748) (end 91.034321 117.697472) (stroke (width 0.05) (type default))
  (layer "Edge.Cuts"))
 (gr_line (start 142.839961 117.54305) (end 142.80736 94.582424) (stroke (width 0.05) (type default)) (layer "Edge.Cuts"))
 (gr_arc (start 91.059 94.181422) (mid 91.302549 93.5736) (end 91.905789 93.318914) (stroke (width 0.05) (type default)) (layer "Edge.Cuts"))
 (gr_line (start 91.905789 93.319607) (end 141.63196 93.435419) (stroke (width 0.05) (type default)) (layer "Edge.Cuts"))
 (segment (start 113.13 96.2) (end 112.8 95.87) (width 0.2) (layer "F.Cu") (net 5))
 (segment (start 139.3 104.4) (end 139.3 101.89) (width 0.2) (layer "F.Cu") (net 5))
 (segment (start 121.75 107.95) (end 113.03 107.95) (width 0.2) (layer "F.Cu") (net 5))
 (segment (start 94.7 99) (end 97.4 101.7) (width 0.2) (layer "F.Cu") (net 5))
 (segment (start 94.7 96.4) (end 94.7 99) (width 0.2) (layer "F.Cu") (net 5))
 (segment (start 138.9 104.8) (end 139.3 104.4) (width 0.2) (layer "F.Cu") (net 5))
 (segment (start 140.52 114.485) (end 140.97 114.935) (width 0.2) (layer "F.Cu") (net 5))
 (segment (start 136.525 108.615) (end 136.525 105.875) (width 0.2) (layer "F.Cu") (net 5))
 (segment (start 136.525 105.875) (end 136.7 105.7) (width 0.2) (layer "F.Cu") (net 5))
 (segment (start 111.63 94.7) (end 96.4 94.7) (width 0.2) (layer "F.Cu") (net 5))
 (segment (start 96.4 94.7) (end 94.7 96.4) (width 0.2) (layer "F.Cu") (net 5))
 (segment (start 112.8 95.87) (end 111.63 94.7) (width 0.2) (layer "F.Cu") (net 5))
 (segment (start 125.1 111.3) (end 121.75 107.95) (width 0.2) (layer "F.Cu") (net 5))
 (segment (start 136.525 110.49) (end 136.525 108.615) (width 0.2) (layer "F.Cu") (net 5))
 (segment (start 140.52 112.3) (end 140.52 114.485) (width 0.2) (layer "F.Cu") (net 5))
 (segment (start 140.97 114.935) (end 136.525 110.49) (width 0.2) (layer "F.Cu") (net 5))
 (via (at 136.7 105.7) (size 0.6) (drill 0.3) (layers "F.Cu" "B.Cu") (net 5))
 (via (at 138.9 104.8) (size 0.6) (drill 0.3) (layers "F.Cu" "B.Cu") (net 5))
 (segment (start 125.1 111.3) (end 125.1 114.5) (width 0.2) (layer "B.Cu") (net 5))
 (segment (start 138.308617 117.596383) (end 140.97 114.935) (width 0.2) (layer "B.Cu") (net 5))
 (segment (start 136.7 105.7) (end 138 105.7) (width 0.2) (layer "B.Cu") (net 5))
 (segment (start 125.1 114.5) (end 128.196383 117.596383) (width 0.2) (layer "B.Cu") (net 5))
 (segment (start 111.599 97.071) (end 111.599 106.519) (width 0.2) (layer "B.Cu") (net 5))
 (segment (start 138 105.7) (end 138.9 104.8) (width 0.2) (layer "B.Cu") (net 5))
 (segment (start 128.196383 117.596383) (end 138.308617 117.596383) (width 0.2) (layer "B.Cu") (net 5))
 (segment (start 112.8 95.87) (end 111.599 97.071) (width 0.2) (layer "B.Cu") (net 5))
 (segment (start 111.599 106.519) (end 113.03 107.95) (width 0.2) (layer "B.Cu") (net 5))
 (segment (start 110.85 111.3) (end 120.1 111.3) (width 0.2) (layer "F.Cu") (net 3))
 (segment (start 129.339 112.401) (end 130.1 113.162) (width 0.2) (layer "F.Cu") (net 3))
 (segment (start 121.201 112.401) (end 129.339 112.401) (width 0.2) (layer "F.Cu") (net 3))
 (segment (start 105.01 95.99) (end 104.3 96.7) (width 0.2) (layer "F.Cu") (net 3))
 (segment (start 130.1 113.162) (end 130.1 115.68) (width 0.2) (layer "F.Cu") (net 3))
 (segment (start 120.1 111.3) (end 121.201 112.401) (width 0.2) (layer "F.Cu") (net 3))
 (segment (start 107.5 107.95) (end 105.15 107.95) (width 0.2) (layer "F.Cu") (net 3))
 (segment (start 105.15 107.95) (end 104.3 107.1) (width 0.2) (layer "F.Cu") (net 3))
 (segment (start 107 95.99) (end 105.01 95.99) (width 0.2) (layer "F.Cu") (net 3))
 (segment (start 107.5 107.95) (end 110.85 111.3) (width 0.2) (layer "F.Cu") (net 3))
 (segment (start 129.339 112.401) (end 133.125 108.615) (width 0.2) (layer "F.Cu") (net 3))
 (via (at 104.3 107.1) (size 0.6) (drill 0.3) (layers "F.Cu" "B.Cu") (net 3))
 (via (at 104.3 96.7) (size 0.6) (drill 0.3) (layers "F.Cu" "B.Cu") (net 3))
 (segment (start 104.3 96.7) (end 104.3 107.1) (width 0.2) (layer "B.Cu") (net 3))
 (segment (start 101.9 101.2) (end 121.3 101.2) (width 0.2) (layer "F.Cu") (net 8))
 (segment (start 97.4 96.7) (end 101.9 101.2) (width 0.2) (layer "F.Cu") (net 8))
 (segment (start 127.9 104.725) (end 128.585 105.41) (width 0.2) (layer "F.Cu") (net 8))
 (segment (start 122.92 102.82) (end 127.9 102.82) (width 0.2) (layer "F.Cu") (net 8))
 (segment (start 127.9 102.82) (end 127.9 104.725) (width 0.2) (layer "F.Cu") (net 8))
 (segment (start 121.3 101.2) (end 122.92 102.82) (width 0.2) (layer "F.Cu") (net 8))
 (segment (start 96.6 114.895) (end 106.825 114.895) (width 0.2) (layer "F.Cu") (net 2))
 (segment (start 106.825 114.895) (end 107.5 115.57) (width 0.2) (layer "F.Cu") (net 2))
 (segment (start 107.5 115.57) (end 113.03 115.57) (width 0.2) (layer "F.Cu") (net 2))
 (segment (start 102.885 103.61) (end 96.6 109.895) (width 0.2) (layer "F.Cu") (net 1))
 (segment (start 112.68 103.61) (end 112.8 103.49) (width 0.2) (layer "F.Cu") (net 1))
 (segment (start 107 103.61) (end 102.885 103.61) (width 0.2) (layer "F.Cu") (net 1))
 (segment (start 107 103.61) (end 112.68 103.61) (width 0.2) (layer "F.Cu") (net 1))
 (segment (start 134.825 108.615) (end 134.825 113.46) (width 0.2) (layer "F.Cu") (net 4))
 (segment (start 134.825 108.615) (end 134.825 106.315) (width 0.2) (layer "F.Cu") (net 4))
 (segment (start 134.825 106.315) (end 133.92 105.41) (width 0.2) (layer "F.Cu") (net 4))
 (segment (start 134.825 113.46) (end 133.35 114.935) (width 0.2) (layer "F.Cu") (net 4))
 (segment (start 133.92 105.41) (end 129.225 105.41) (width 0.2) (layer "F.Cu") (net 4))
 (segment (start 138.225 108.615) (end 138.225 106.315) (width 0.2) (layer "F.Cu") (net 6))
 (segment (start 128.099999 102.18) (end 127.9 102.18) (width 0.2) (layer "F.Cu") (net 6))
 (segment (start 136.376 104.466) (end 130.385999 104.466) (width 0.2) (layer "F.Cu") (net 6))
 (segment (start 127.9 102.18) (end 127.8 102.08) (width 0.2) (layer "F.Cu") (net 6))
 (segment (start 127.18 102.08) (end 121.3 96.2) (width 0.2) (layer "F.Cu") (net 6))
 (segment (start 127.8 102.08) (end 127.18 102.08) (width 0.2) (layer "F.Cu") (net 6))
 (segment (start 138.225 110.645) (end 138.225 108.615) (width 0.2) (layer "F.Cu") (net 6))
 (segment (start 138.225 106.315) (end 136.376 104.466) (width 0.2) (layer "F.Cu") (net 6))
 (segment (start 130.385999 104.466) (end 128.099999 102.18) (width 0.2) (layer "F.Cu") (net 6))
 (segment (start 139.88 112.3) (end 138.225 110.645) (width 0.2) (layer "F.Cu") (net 6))
 (segment (start 141.283471 116.32) (end 142.171 115.432471) (width 0.2) (layer "F.Cu") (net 7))
 (segment (start 142.171 115.432471) (end 142.171 110.861) (width 0.2) (layer "F.Cu") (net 7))
 (segment (start 130.1 116.32) (end 141.283471 116.32) (width 0.2) (layer "F.Cu") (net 7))
 (segment (start 142.171 110.861) (end 139.925 108.615) (width 0.2) (layer "F.Cu") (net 7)))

